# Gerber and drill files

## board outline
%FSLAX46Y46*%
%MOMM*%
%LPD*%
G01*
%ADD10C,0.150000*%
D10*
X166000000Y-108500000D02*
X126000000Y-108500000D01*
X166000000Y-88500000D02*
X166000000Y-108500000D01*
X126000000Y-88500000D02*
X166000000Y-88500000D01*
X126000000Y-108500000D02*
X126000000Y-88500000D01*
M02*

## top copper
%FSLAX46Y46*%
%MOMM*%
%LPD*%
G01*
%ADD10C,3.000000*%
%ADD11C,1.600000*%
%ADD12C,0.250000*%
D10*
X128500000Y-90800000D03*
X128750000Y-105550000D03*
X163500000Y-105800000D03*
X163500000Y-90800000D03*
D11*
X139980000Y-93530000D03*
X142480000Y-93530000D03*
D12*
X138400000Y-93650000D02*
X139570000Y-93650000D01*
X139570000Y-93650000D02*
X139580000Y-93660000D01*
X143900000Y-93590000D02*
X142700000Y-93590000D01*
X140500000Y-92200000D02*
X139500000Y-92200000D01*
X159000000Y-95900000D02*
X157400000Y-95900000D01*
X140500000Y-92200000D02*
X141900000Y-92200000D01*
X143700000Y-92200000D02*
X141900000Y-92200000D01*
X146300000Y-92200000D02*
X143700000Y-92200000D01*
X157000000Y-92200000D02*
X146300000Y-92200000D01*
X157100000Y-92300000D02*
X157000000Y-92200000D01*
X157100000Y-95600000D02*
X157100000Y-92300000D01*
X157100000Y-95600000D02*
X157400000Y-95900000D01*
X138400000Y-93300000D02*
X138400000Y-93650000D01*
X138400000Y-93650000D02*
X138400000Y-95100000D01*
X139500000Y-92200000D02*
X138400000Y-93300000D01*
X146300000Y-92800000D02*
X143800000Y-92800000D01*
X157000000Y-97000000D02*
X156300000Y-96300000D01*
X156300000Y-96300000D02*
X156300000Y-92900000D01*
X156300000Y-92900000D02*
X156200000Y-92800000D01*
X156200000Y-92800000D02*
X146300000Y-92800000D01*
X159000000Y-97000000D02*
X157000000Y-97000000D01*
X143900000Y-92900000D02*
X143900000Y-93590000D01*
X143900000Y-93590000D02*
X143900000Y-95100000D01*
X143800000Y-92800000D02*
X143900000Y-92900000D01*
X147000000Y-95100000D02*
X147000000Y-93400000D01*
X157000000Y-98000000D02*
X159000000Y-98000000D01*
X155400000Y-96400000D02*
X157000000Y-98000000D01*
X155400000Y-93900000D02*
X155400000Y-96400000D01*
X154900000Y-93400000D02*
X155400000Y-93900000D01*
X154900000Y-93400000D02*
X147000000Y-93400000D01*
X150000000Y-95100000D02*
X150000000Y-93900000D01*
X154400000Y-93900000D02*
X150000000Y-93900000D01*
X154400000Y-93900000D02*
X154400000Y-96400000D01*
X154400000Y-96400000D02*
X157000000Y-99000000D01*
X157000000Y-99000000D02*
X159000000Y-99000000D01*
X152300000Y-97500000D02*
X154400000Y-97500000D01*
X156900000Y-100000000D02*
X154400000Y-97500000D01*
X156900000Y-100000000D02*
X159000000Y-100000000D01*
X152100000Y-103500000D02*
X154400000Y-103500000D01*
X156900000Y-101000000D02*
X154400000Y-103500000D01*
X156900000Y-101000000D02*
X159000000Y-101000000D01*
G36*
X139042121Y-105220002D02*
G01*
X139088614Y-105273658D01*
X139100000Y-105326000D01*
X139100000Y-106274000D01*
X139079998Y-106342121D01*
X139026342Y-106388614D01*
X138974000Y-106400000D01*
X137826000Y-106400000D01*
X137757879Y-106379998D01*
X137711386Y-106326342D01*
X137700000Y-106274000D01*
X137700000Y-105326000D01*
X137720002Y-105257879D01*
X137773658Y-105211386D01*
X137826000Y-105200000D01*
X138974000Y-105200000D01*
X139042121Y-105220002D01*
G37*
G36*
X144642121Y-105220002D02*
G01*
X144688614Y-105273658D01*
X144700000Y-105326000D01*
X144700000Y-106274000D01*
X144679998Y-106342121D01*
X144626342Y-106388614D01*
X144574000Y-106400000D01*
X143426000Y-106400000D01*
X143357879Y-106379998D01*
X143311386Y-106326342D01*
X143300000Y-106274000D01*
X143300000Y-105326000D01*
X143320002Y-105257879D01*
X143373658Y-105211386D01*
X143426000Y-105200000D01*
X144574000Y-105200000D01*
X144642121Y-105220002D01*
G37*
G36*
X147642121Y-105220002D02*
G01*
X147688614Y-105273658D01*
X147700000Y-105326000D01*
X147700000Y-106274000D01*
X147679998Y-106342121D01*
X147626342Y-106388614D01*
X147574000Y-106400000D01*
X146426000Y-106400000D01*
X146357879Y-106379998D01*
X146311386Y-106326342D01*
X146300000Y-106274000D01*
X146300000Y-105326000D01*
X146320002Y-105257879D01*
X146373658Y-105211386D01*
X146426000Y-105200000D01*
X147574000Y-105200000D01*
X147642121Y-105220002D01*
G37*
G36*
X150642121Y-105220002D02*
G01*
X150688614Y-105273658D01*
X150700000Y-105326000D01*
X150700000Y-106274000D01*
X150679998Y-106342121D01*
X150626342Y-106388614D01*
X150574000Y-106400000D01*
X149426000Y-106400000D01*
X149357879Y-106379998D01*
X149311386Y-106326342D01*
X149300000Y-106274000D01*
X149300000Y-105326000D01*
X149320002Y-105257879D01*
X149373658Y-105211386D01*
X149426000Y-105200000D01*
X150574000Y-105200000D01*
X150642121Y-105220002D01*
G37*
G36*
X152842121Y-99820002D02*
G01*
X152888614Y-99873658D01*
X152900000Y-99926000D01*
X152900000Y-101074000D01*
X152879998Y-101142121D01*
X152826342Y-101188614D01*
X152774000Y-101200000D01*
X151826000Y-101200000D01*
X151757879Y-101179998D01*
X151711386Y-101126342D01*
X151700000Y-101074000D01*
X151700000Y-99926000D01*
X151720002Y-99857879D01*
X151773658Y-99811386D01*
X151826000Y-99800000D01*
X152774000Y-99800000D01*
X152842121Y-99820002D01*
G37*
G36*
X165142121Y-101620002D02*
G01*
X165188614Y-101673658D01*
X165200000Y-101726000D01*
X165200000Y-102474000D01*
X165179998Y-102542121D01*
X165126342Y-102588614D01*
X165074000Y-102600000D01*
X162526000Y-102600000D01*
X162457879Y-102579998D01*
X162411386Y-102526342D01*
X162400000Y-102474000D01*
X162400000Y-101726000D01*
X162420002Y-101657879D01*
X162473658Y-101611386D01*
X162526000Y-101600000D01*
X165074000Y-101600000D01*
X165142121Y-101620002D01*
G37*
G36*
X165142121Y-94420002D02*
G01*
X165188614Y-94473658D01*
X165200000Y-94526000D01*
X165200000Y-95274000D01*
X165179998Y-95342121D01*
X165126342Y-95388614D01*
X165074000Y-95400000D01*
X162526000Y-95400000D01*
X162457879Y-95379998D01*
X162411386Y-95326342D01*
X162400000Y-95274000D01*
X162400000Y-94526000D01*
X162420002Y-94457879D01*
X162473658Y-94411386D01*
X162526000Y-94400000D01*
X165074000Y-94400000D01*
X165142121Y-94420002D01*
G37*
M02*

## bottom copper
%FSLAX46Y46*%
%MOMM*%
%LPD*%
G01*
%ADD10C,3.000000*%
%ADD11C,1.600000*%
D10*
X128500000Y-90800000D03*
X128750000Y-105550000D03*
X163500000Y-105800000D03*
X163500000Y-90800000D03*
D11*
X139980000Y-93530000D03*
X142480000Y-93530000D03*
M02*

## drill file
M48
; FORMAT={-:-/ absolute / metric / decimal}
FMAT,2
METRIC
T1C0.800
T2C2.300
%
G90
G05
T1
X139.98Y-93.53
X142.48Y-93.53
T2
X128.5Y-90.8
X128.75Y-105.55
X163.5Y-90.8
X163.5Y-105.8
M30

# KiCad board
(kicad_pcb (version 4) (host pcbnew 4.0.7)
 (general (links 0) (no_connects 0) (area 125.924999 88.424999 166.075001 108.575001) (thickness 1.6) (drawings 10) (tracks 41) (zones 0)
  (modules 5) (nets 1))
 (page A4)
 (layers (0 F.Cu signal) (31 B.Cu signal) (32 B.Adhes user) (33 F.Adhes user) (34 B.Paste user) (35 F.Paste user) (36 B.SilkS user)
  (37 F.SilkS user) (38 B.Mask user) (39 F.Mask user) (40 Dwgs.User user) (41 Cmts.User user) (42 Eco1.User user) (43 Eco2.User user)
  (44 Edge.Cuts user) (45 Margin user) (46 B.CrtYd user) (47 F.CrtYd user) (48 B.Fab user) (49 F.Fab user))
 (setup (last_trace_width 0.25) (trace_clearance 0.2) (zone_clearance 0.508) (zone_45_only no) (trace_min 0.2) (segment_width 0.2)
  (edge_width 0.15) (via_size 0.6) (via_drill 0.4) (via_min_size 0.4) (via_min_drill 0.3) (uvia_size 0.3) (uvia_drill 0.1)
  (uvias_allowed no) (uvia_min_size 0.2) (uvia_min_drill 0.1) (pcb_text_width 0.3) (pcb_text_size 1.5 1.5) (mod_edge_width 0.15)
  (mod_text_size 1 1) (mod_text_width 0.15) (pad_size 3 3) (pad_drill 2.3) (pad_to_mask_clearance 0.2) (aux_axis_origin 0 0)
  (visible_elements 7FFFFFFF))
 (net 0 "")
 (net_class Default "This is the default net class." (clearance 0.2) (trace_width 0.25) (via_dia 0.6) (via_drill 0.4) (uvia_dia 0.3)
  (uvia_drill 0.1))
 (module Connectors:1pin (layer F.Cu) (at 128.5 90.8)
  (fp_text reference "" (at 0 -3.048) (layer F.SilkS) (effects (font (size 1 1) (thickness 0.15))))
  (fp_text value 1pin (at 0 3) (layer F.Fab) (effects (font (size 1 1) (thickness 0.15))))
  (pad 1 thru_hole circle (at 0 0) (size 3 3) (drill 2.3) (layers *.Cu *.Mask)))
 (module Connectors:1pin (layer F.Cu) (at 128.75 105.55)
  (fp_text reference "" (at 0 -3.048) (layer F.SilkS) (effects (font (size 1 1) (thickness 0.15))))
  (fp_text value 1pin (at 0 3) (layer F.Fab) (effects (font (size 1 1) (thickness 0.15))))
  (pad 1 thru_hole circle (at 0 0) (size 3 3) (drill 2.3) (layers *.Cu *.Mask)))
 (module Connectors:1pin (layer F.Cu) (at 163.5 105.8)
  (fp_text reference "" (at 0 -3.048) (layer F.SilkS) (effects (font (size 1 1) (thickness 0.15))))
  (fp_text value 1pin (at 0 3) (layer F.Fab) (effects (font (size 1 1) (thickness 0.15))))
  (pad 1 thru_hole circle (at 0 0) (size 3 3) (drill 2.3) (layers *.Cu *.Mask)))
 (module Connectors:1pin (layer F.Cu) (at 163.5 90.8)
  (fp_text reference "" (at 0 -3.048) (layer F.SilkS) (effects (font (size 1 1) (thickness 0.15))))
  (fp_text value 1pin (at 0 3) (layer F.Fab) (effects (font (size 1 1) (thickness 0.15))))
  (pad 1 thru_hole circle (at 0 0) (size 3 3) (drill 2.3) (layers *.Cu *.Mask)))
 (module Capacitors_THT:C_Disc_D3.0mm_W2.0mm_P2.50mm (layer F.Cu) (at 139.98 93.53)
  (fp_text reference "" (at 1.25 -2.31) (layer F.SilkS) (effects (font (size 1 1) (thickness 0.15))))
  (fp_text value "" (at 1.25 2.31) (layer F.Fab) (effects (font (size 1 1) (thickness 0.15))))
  (pad 1 thru_hole circle (at 0 0) (size 1.6 1.6) (drill 0.8) (layers *.Cu *.Mask))
  (pad 2 thru_hole circle (at 2.5 0) (size 1.6 1.6) (drill 0.8) (layers *.Cu *.Mask)))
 (gr_line (start 166 108.5) (end 126 108.5) (angle 90) (layer Edge.Cuts) (width 0.15))
 (gr_line (start 166 88.5) (end 166 108.5) (angle 90) (layer Edge.Cuts) (width 0.15))
 (gr_line (start 126 88.5) (end 166 88.5) (angle 90) (layer Edge.Cuts) (width 0.15))
 (gr_line (start 126 108.5) (end 126 88.5) (angle 90) (layer Edge.Cuts) (width 0.15))
 (segment (start 138.4 93.65) (end 139.57 93.65) (width 0.25) (layer F.Cu) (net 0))
 (segment (start 139.57 93.65) (end 139.58 93.66) (width 0.25) (layer F.Cu) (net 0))
 (segment (start 143.9 93.59) (end 142.7 93.59) (width 0.25) (layer F.Cu) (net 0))
 (segment (start 140.5 92.2) (end 139.5 92.2) (width 0.25) (layer F.Cu) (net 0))
 (segment (start 159 95.9) (end 157.4 95.9) (width 0.25) (layer F.Cu) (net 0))
 (segment (start 140.5 92.2) (end 141.9 92.2) (width 0.25) (layer F.Cu) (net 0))
 (segment (start 143.7 92.2) (end 141.9 92.2) (width 0.25) (layer F.Cu) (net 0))
 (segment (start 146.3 92.2) (end 143.7 92.2) (width 0.25) (layer F.Cu) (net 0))
 (segment (start 157 92.2) (end 146.3 92.2) (width 0.25) (layer F.Cu) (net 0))
 (segment (start 157.1 92.3) (end 157 92.2) (width 0.25) (layer F.Cu) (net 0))
 (segment (start 157.1 95.6) (end 157.1 92.3) (width 0.25) (layer F.Cu) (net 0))
 (segment (start 157.1 95.6) (end 157.4 95.9) (width 0.25) (layer F.Cu) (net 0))
 (segment (start 138.4 93.3) (end 138.4 93.65) (width 0.25) (layer F.Cu) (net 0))
 (segment (start 138.4 93.65) (end 138.4 95.1) (width 0.25) (layer F.Cu) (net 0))
 (segment (start 139.5 92.2) (end 138.4 93.3) (width 0.25) (layer F.Cu) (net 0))
 (segment (start 146.3 92.8) (end 143.8 92.8) (width 0.25) (layer F.Cu) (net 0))
 (segment (start 157 97) (end 156.3 96.3) (width 0.25) (layer F.Cu) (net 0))
 (segment (start 156.3 96.3) (end 156.3 92.9) (width 0.25) (layer F.Cu) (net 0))
 (segment (start 156.3 92.9) (end 156.2 92.8) (width 0.25) (layer F.Cu) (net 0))
 (segment (start 156.2 92.8) (end 146.3 92.8) (width 0.25) (layer F.Cu) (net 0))
 (segment (start 159 97) (end 157 97) (width 0.25) (layer F.Cu) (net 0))
 (segment (start 143.9 92.9) (end 143.9 93.59) (width 0.25) (layer F.Cu) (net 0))
 (segment (start 143.9 93.59) (end 143.9 95.1) (width 0.25) (layer F.Cu) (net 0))
 (segment (start 143.8 92.8) (end 143.9 92.9) (width 0.25) (layer F.Cu) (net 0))
 (segment (start 147 95.1) (end 147 93.4) (width 0.25) (layer F.Cu) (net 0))
 (segment (start 157 98) (end 159 98) (width 0.25) (layer F.Cu) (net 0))
 (segment (start 155.4 96.4) (end 157 98) (width 0.25) (layer F.Cu) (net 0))
 (segment (start 155.4 93.9) (end 155.4 96.4) (width 0.25) (layer F.Cu) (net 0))
 (segment (start 154.9 93.4) (end 155.4 93.9) (width 0.25) (layer F.Cu) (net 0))
 (segment (start 154.9 93.4) (end 147 93.4) (width 0.25) (layer F.Cu) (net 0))
 (segment (start 150 95.1) (end 150 93.9) (width 0.25) (layer F.Cu) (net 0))
 (segment (start 154.4 93.9) (end 150 93.9) (width 0.25) (layer F.Cu) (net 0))
 (segment (start 154.4 93.9) (end 154.4 96.4) (width 0.25) (layer F.Cu) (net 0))
 (segment (start 154.4 96.4) (end 157 99) (width 0.25) (layer F.Cu) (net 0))
 (segment (start 157 99) (end 159 99) (width 0.25) (layer F.Cu) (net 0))
 (segment (start 152.3 97.5) (end 154.4 97.5) (width 0.25) (layer F.Cu) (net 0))
 (segment (start 156.9 100) (end 154.4 97.5) (width 0.25) (layer F.Cu) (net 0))
 (segment (start 156.9 100) (end 159 100) (width 0.25) (layer F.Cu) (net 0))
 (segment (start 152.1 103.5) (end 154.4 103.5) (width 0.25) (layer F.Cu) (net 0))
 (segment (start 156.9 101) (end 154.4 103.5) (width 0.25) (layer F.Cu) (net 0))
 (segment (start 156.9 101) (end 159 101) (width 0.25) (layer F.Cu) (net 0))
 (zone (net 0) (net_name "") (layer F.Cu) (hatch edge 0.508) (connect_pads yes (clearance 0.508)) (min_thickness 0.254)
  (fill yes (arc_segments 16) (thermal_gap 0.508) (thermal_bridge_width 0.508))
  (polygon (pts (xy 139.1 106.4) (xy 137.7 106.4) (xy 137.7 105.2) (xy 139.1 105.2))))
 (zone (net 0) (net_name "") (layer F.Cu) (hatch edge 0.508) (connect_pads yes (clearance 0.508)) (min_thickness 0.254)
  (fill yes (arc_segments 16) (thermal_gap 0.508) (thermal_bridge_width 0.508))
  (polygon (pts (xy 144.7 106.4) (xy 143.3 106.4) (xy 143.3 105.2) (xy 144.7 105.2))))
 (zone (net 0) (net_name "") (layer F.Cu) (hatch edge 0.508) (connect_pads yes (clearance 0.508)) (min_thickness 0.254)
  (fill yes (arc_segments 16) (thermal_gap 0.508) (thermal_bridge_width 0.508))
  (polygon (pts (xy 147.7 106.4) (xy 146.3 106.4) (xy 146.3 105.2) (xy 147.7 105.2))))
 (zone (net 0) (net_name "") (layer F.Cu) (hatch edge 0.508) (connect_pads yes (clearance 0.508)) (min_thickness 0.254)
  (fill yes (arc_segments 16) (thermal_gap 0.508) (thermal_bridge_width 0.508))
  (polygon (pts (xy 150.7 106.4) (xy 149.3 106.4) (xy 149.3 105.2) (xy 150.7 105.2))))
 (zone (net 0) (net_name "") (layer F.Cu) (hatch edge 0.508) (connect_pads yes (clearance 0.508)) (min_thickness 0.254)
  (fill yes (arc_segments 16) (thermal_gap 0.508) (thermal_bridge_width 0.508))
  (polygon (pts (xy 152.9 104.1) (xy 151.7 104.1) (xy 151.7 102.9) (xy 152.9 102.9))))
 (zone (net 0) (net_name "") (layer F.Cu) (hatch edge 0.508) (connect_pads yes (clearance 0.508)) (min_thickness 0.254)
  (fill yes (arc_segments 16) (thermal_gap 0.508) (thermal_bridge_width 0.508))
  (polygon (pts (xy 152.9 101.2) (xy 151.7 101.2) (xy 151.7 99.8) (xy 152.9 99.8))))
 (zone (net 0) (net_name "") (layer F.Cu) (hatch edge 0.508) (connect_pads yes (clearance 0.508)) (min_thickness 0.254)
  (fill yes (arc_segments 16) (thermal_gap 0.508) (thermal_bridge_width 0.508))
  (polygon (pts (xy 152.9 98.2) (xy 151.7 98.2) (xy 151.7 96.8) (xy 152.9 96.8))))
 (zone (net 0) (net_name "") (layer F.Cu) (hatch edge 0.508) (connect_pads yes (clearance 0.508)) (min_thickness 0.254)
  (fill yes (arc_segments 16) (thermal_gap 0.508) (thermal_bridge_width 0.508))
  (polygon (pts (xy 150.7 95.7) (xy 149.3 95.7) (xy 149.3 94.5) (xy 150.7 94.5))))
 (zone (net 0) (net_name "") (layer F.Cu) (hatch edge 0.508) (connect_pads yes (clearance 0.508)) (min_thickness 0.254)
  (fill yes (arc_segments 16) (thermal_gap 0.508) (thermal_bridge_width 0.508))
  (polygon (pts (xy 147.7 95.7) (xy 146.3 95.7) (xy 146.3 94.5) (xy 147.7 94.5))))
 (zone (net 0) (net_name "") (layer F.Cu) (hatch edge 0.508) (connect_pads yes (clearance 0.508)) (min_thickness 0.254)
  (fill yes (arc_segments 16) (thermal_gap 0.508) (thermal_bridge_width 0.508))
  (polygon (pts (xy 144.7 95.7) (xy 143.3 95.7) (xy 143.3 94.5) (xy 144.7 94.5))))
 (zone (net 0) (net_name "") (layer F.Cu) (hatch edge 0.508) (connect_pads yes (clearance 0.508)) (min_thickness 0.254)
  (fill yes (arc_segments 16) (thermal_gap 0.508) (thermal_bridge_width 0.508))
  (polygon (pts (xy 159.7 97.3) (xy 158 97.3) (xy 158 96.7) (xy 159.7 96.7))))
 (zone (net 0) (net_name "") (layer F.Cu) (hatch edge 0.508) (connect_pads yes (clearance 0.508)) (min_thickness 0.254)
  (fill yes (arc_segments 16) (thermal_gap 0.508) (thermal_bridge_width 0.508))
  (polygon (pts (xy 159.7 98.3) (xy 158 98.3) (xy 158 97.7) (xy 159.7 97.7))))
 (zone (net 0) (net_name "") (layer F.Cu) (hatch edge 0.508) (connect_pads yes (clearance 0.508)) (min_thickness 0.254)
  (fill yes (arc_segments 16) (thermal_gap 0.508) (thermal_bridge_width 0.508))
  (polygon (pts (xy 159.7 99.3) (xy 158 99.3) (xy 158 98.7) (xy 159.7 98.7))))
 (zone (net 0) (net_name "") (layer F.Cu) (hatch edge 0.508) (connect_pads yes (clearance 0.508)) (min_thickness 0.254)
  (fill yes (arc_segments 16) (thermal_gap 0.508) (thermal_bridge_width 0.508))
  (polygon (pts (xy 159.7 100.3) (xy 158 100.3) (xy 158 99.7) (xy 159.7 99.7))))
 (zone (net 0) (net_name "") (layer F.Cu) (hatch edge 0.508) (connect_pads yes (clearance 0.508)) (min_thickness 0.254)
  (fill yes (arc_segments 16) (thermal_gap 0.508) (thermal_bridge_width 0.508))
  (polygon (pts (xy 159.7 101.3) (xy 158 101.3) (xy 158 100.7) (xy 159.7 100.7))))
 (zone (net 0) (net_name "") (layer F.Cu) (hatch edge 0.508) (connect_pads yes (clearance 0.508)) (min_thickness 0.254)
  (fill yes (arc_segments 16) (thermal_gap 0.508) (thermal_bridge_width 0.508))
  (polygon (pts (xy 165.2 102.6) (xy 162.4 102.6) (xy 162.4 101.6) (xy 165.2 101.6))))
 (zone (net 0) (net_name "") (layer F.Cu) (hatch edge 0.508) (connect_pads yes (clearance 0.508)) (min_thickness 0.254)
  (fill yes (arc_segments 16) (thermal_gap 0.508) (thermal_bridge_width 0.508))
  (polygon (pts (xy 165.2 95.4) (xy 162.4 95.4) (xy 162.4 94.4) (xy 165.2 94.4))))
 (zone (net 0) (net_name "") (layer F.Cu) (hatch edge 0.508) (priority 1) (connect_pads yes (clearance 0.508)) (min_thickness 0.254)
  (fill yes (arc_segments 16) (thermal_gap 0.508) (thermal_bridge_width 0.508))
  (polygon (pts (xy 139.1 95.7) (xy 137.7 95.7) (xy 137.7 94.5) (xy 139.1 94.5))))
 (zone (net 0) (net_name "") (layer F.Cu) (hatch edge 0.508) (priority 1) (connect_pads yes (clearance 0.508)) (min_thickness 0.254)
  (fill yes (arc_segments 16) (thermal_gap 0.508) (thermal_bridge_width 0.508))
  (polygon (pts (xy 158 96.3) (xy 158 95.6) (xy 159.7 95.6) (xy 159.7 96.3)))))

